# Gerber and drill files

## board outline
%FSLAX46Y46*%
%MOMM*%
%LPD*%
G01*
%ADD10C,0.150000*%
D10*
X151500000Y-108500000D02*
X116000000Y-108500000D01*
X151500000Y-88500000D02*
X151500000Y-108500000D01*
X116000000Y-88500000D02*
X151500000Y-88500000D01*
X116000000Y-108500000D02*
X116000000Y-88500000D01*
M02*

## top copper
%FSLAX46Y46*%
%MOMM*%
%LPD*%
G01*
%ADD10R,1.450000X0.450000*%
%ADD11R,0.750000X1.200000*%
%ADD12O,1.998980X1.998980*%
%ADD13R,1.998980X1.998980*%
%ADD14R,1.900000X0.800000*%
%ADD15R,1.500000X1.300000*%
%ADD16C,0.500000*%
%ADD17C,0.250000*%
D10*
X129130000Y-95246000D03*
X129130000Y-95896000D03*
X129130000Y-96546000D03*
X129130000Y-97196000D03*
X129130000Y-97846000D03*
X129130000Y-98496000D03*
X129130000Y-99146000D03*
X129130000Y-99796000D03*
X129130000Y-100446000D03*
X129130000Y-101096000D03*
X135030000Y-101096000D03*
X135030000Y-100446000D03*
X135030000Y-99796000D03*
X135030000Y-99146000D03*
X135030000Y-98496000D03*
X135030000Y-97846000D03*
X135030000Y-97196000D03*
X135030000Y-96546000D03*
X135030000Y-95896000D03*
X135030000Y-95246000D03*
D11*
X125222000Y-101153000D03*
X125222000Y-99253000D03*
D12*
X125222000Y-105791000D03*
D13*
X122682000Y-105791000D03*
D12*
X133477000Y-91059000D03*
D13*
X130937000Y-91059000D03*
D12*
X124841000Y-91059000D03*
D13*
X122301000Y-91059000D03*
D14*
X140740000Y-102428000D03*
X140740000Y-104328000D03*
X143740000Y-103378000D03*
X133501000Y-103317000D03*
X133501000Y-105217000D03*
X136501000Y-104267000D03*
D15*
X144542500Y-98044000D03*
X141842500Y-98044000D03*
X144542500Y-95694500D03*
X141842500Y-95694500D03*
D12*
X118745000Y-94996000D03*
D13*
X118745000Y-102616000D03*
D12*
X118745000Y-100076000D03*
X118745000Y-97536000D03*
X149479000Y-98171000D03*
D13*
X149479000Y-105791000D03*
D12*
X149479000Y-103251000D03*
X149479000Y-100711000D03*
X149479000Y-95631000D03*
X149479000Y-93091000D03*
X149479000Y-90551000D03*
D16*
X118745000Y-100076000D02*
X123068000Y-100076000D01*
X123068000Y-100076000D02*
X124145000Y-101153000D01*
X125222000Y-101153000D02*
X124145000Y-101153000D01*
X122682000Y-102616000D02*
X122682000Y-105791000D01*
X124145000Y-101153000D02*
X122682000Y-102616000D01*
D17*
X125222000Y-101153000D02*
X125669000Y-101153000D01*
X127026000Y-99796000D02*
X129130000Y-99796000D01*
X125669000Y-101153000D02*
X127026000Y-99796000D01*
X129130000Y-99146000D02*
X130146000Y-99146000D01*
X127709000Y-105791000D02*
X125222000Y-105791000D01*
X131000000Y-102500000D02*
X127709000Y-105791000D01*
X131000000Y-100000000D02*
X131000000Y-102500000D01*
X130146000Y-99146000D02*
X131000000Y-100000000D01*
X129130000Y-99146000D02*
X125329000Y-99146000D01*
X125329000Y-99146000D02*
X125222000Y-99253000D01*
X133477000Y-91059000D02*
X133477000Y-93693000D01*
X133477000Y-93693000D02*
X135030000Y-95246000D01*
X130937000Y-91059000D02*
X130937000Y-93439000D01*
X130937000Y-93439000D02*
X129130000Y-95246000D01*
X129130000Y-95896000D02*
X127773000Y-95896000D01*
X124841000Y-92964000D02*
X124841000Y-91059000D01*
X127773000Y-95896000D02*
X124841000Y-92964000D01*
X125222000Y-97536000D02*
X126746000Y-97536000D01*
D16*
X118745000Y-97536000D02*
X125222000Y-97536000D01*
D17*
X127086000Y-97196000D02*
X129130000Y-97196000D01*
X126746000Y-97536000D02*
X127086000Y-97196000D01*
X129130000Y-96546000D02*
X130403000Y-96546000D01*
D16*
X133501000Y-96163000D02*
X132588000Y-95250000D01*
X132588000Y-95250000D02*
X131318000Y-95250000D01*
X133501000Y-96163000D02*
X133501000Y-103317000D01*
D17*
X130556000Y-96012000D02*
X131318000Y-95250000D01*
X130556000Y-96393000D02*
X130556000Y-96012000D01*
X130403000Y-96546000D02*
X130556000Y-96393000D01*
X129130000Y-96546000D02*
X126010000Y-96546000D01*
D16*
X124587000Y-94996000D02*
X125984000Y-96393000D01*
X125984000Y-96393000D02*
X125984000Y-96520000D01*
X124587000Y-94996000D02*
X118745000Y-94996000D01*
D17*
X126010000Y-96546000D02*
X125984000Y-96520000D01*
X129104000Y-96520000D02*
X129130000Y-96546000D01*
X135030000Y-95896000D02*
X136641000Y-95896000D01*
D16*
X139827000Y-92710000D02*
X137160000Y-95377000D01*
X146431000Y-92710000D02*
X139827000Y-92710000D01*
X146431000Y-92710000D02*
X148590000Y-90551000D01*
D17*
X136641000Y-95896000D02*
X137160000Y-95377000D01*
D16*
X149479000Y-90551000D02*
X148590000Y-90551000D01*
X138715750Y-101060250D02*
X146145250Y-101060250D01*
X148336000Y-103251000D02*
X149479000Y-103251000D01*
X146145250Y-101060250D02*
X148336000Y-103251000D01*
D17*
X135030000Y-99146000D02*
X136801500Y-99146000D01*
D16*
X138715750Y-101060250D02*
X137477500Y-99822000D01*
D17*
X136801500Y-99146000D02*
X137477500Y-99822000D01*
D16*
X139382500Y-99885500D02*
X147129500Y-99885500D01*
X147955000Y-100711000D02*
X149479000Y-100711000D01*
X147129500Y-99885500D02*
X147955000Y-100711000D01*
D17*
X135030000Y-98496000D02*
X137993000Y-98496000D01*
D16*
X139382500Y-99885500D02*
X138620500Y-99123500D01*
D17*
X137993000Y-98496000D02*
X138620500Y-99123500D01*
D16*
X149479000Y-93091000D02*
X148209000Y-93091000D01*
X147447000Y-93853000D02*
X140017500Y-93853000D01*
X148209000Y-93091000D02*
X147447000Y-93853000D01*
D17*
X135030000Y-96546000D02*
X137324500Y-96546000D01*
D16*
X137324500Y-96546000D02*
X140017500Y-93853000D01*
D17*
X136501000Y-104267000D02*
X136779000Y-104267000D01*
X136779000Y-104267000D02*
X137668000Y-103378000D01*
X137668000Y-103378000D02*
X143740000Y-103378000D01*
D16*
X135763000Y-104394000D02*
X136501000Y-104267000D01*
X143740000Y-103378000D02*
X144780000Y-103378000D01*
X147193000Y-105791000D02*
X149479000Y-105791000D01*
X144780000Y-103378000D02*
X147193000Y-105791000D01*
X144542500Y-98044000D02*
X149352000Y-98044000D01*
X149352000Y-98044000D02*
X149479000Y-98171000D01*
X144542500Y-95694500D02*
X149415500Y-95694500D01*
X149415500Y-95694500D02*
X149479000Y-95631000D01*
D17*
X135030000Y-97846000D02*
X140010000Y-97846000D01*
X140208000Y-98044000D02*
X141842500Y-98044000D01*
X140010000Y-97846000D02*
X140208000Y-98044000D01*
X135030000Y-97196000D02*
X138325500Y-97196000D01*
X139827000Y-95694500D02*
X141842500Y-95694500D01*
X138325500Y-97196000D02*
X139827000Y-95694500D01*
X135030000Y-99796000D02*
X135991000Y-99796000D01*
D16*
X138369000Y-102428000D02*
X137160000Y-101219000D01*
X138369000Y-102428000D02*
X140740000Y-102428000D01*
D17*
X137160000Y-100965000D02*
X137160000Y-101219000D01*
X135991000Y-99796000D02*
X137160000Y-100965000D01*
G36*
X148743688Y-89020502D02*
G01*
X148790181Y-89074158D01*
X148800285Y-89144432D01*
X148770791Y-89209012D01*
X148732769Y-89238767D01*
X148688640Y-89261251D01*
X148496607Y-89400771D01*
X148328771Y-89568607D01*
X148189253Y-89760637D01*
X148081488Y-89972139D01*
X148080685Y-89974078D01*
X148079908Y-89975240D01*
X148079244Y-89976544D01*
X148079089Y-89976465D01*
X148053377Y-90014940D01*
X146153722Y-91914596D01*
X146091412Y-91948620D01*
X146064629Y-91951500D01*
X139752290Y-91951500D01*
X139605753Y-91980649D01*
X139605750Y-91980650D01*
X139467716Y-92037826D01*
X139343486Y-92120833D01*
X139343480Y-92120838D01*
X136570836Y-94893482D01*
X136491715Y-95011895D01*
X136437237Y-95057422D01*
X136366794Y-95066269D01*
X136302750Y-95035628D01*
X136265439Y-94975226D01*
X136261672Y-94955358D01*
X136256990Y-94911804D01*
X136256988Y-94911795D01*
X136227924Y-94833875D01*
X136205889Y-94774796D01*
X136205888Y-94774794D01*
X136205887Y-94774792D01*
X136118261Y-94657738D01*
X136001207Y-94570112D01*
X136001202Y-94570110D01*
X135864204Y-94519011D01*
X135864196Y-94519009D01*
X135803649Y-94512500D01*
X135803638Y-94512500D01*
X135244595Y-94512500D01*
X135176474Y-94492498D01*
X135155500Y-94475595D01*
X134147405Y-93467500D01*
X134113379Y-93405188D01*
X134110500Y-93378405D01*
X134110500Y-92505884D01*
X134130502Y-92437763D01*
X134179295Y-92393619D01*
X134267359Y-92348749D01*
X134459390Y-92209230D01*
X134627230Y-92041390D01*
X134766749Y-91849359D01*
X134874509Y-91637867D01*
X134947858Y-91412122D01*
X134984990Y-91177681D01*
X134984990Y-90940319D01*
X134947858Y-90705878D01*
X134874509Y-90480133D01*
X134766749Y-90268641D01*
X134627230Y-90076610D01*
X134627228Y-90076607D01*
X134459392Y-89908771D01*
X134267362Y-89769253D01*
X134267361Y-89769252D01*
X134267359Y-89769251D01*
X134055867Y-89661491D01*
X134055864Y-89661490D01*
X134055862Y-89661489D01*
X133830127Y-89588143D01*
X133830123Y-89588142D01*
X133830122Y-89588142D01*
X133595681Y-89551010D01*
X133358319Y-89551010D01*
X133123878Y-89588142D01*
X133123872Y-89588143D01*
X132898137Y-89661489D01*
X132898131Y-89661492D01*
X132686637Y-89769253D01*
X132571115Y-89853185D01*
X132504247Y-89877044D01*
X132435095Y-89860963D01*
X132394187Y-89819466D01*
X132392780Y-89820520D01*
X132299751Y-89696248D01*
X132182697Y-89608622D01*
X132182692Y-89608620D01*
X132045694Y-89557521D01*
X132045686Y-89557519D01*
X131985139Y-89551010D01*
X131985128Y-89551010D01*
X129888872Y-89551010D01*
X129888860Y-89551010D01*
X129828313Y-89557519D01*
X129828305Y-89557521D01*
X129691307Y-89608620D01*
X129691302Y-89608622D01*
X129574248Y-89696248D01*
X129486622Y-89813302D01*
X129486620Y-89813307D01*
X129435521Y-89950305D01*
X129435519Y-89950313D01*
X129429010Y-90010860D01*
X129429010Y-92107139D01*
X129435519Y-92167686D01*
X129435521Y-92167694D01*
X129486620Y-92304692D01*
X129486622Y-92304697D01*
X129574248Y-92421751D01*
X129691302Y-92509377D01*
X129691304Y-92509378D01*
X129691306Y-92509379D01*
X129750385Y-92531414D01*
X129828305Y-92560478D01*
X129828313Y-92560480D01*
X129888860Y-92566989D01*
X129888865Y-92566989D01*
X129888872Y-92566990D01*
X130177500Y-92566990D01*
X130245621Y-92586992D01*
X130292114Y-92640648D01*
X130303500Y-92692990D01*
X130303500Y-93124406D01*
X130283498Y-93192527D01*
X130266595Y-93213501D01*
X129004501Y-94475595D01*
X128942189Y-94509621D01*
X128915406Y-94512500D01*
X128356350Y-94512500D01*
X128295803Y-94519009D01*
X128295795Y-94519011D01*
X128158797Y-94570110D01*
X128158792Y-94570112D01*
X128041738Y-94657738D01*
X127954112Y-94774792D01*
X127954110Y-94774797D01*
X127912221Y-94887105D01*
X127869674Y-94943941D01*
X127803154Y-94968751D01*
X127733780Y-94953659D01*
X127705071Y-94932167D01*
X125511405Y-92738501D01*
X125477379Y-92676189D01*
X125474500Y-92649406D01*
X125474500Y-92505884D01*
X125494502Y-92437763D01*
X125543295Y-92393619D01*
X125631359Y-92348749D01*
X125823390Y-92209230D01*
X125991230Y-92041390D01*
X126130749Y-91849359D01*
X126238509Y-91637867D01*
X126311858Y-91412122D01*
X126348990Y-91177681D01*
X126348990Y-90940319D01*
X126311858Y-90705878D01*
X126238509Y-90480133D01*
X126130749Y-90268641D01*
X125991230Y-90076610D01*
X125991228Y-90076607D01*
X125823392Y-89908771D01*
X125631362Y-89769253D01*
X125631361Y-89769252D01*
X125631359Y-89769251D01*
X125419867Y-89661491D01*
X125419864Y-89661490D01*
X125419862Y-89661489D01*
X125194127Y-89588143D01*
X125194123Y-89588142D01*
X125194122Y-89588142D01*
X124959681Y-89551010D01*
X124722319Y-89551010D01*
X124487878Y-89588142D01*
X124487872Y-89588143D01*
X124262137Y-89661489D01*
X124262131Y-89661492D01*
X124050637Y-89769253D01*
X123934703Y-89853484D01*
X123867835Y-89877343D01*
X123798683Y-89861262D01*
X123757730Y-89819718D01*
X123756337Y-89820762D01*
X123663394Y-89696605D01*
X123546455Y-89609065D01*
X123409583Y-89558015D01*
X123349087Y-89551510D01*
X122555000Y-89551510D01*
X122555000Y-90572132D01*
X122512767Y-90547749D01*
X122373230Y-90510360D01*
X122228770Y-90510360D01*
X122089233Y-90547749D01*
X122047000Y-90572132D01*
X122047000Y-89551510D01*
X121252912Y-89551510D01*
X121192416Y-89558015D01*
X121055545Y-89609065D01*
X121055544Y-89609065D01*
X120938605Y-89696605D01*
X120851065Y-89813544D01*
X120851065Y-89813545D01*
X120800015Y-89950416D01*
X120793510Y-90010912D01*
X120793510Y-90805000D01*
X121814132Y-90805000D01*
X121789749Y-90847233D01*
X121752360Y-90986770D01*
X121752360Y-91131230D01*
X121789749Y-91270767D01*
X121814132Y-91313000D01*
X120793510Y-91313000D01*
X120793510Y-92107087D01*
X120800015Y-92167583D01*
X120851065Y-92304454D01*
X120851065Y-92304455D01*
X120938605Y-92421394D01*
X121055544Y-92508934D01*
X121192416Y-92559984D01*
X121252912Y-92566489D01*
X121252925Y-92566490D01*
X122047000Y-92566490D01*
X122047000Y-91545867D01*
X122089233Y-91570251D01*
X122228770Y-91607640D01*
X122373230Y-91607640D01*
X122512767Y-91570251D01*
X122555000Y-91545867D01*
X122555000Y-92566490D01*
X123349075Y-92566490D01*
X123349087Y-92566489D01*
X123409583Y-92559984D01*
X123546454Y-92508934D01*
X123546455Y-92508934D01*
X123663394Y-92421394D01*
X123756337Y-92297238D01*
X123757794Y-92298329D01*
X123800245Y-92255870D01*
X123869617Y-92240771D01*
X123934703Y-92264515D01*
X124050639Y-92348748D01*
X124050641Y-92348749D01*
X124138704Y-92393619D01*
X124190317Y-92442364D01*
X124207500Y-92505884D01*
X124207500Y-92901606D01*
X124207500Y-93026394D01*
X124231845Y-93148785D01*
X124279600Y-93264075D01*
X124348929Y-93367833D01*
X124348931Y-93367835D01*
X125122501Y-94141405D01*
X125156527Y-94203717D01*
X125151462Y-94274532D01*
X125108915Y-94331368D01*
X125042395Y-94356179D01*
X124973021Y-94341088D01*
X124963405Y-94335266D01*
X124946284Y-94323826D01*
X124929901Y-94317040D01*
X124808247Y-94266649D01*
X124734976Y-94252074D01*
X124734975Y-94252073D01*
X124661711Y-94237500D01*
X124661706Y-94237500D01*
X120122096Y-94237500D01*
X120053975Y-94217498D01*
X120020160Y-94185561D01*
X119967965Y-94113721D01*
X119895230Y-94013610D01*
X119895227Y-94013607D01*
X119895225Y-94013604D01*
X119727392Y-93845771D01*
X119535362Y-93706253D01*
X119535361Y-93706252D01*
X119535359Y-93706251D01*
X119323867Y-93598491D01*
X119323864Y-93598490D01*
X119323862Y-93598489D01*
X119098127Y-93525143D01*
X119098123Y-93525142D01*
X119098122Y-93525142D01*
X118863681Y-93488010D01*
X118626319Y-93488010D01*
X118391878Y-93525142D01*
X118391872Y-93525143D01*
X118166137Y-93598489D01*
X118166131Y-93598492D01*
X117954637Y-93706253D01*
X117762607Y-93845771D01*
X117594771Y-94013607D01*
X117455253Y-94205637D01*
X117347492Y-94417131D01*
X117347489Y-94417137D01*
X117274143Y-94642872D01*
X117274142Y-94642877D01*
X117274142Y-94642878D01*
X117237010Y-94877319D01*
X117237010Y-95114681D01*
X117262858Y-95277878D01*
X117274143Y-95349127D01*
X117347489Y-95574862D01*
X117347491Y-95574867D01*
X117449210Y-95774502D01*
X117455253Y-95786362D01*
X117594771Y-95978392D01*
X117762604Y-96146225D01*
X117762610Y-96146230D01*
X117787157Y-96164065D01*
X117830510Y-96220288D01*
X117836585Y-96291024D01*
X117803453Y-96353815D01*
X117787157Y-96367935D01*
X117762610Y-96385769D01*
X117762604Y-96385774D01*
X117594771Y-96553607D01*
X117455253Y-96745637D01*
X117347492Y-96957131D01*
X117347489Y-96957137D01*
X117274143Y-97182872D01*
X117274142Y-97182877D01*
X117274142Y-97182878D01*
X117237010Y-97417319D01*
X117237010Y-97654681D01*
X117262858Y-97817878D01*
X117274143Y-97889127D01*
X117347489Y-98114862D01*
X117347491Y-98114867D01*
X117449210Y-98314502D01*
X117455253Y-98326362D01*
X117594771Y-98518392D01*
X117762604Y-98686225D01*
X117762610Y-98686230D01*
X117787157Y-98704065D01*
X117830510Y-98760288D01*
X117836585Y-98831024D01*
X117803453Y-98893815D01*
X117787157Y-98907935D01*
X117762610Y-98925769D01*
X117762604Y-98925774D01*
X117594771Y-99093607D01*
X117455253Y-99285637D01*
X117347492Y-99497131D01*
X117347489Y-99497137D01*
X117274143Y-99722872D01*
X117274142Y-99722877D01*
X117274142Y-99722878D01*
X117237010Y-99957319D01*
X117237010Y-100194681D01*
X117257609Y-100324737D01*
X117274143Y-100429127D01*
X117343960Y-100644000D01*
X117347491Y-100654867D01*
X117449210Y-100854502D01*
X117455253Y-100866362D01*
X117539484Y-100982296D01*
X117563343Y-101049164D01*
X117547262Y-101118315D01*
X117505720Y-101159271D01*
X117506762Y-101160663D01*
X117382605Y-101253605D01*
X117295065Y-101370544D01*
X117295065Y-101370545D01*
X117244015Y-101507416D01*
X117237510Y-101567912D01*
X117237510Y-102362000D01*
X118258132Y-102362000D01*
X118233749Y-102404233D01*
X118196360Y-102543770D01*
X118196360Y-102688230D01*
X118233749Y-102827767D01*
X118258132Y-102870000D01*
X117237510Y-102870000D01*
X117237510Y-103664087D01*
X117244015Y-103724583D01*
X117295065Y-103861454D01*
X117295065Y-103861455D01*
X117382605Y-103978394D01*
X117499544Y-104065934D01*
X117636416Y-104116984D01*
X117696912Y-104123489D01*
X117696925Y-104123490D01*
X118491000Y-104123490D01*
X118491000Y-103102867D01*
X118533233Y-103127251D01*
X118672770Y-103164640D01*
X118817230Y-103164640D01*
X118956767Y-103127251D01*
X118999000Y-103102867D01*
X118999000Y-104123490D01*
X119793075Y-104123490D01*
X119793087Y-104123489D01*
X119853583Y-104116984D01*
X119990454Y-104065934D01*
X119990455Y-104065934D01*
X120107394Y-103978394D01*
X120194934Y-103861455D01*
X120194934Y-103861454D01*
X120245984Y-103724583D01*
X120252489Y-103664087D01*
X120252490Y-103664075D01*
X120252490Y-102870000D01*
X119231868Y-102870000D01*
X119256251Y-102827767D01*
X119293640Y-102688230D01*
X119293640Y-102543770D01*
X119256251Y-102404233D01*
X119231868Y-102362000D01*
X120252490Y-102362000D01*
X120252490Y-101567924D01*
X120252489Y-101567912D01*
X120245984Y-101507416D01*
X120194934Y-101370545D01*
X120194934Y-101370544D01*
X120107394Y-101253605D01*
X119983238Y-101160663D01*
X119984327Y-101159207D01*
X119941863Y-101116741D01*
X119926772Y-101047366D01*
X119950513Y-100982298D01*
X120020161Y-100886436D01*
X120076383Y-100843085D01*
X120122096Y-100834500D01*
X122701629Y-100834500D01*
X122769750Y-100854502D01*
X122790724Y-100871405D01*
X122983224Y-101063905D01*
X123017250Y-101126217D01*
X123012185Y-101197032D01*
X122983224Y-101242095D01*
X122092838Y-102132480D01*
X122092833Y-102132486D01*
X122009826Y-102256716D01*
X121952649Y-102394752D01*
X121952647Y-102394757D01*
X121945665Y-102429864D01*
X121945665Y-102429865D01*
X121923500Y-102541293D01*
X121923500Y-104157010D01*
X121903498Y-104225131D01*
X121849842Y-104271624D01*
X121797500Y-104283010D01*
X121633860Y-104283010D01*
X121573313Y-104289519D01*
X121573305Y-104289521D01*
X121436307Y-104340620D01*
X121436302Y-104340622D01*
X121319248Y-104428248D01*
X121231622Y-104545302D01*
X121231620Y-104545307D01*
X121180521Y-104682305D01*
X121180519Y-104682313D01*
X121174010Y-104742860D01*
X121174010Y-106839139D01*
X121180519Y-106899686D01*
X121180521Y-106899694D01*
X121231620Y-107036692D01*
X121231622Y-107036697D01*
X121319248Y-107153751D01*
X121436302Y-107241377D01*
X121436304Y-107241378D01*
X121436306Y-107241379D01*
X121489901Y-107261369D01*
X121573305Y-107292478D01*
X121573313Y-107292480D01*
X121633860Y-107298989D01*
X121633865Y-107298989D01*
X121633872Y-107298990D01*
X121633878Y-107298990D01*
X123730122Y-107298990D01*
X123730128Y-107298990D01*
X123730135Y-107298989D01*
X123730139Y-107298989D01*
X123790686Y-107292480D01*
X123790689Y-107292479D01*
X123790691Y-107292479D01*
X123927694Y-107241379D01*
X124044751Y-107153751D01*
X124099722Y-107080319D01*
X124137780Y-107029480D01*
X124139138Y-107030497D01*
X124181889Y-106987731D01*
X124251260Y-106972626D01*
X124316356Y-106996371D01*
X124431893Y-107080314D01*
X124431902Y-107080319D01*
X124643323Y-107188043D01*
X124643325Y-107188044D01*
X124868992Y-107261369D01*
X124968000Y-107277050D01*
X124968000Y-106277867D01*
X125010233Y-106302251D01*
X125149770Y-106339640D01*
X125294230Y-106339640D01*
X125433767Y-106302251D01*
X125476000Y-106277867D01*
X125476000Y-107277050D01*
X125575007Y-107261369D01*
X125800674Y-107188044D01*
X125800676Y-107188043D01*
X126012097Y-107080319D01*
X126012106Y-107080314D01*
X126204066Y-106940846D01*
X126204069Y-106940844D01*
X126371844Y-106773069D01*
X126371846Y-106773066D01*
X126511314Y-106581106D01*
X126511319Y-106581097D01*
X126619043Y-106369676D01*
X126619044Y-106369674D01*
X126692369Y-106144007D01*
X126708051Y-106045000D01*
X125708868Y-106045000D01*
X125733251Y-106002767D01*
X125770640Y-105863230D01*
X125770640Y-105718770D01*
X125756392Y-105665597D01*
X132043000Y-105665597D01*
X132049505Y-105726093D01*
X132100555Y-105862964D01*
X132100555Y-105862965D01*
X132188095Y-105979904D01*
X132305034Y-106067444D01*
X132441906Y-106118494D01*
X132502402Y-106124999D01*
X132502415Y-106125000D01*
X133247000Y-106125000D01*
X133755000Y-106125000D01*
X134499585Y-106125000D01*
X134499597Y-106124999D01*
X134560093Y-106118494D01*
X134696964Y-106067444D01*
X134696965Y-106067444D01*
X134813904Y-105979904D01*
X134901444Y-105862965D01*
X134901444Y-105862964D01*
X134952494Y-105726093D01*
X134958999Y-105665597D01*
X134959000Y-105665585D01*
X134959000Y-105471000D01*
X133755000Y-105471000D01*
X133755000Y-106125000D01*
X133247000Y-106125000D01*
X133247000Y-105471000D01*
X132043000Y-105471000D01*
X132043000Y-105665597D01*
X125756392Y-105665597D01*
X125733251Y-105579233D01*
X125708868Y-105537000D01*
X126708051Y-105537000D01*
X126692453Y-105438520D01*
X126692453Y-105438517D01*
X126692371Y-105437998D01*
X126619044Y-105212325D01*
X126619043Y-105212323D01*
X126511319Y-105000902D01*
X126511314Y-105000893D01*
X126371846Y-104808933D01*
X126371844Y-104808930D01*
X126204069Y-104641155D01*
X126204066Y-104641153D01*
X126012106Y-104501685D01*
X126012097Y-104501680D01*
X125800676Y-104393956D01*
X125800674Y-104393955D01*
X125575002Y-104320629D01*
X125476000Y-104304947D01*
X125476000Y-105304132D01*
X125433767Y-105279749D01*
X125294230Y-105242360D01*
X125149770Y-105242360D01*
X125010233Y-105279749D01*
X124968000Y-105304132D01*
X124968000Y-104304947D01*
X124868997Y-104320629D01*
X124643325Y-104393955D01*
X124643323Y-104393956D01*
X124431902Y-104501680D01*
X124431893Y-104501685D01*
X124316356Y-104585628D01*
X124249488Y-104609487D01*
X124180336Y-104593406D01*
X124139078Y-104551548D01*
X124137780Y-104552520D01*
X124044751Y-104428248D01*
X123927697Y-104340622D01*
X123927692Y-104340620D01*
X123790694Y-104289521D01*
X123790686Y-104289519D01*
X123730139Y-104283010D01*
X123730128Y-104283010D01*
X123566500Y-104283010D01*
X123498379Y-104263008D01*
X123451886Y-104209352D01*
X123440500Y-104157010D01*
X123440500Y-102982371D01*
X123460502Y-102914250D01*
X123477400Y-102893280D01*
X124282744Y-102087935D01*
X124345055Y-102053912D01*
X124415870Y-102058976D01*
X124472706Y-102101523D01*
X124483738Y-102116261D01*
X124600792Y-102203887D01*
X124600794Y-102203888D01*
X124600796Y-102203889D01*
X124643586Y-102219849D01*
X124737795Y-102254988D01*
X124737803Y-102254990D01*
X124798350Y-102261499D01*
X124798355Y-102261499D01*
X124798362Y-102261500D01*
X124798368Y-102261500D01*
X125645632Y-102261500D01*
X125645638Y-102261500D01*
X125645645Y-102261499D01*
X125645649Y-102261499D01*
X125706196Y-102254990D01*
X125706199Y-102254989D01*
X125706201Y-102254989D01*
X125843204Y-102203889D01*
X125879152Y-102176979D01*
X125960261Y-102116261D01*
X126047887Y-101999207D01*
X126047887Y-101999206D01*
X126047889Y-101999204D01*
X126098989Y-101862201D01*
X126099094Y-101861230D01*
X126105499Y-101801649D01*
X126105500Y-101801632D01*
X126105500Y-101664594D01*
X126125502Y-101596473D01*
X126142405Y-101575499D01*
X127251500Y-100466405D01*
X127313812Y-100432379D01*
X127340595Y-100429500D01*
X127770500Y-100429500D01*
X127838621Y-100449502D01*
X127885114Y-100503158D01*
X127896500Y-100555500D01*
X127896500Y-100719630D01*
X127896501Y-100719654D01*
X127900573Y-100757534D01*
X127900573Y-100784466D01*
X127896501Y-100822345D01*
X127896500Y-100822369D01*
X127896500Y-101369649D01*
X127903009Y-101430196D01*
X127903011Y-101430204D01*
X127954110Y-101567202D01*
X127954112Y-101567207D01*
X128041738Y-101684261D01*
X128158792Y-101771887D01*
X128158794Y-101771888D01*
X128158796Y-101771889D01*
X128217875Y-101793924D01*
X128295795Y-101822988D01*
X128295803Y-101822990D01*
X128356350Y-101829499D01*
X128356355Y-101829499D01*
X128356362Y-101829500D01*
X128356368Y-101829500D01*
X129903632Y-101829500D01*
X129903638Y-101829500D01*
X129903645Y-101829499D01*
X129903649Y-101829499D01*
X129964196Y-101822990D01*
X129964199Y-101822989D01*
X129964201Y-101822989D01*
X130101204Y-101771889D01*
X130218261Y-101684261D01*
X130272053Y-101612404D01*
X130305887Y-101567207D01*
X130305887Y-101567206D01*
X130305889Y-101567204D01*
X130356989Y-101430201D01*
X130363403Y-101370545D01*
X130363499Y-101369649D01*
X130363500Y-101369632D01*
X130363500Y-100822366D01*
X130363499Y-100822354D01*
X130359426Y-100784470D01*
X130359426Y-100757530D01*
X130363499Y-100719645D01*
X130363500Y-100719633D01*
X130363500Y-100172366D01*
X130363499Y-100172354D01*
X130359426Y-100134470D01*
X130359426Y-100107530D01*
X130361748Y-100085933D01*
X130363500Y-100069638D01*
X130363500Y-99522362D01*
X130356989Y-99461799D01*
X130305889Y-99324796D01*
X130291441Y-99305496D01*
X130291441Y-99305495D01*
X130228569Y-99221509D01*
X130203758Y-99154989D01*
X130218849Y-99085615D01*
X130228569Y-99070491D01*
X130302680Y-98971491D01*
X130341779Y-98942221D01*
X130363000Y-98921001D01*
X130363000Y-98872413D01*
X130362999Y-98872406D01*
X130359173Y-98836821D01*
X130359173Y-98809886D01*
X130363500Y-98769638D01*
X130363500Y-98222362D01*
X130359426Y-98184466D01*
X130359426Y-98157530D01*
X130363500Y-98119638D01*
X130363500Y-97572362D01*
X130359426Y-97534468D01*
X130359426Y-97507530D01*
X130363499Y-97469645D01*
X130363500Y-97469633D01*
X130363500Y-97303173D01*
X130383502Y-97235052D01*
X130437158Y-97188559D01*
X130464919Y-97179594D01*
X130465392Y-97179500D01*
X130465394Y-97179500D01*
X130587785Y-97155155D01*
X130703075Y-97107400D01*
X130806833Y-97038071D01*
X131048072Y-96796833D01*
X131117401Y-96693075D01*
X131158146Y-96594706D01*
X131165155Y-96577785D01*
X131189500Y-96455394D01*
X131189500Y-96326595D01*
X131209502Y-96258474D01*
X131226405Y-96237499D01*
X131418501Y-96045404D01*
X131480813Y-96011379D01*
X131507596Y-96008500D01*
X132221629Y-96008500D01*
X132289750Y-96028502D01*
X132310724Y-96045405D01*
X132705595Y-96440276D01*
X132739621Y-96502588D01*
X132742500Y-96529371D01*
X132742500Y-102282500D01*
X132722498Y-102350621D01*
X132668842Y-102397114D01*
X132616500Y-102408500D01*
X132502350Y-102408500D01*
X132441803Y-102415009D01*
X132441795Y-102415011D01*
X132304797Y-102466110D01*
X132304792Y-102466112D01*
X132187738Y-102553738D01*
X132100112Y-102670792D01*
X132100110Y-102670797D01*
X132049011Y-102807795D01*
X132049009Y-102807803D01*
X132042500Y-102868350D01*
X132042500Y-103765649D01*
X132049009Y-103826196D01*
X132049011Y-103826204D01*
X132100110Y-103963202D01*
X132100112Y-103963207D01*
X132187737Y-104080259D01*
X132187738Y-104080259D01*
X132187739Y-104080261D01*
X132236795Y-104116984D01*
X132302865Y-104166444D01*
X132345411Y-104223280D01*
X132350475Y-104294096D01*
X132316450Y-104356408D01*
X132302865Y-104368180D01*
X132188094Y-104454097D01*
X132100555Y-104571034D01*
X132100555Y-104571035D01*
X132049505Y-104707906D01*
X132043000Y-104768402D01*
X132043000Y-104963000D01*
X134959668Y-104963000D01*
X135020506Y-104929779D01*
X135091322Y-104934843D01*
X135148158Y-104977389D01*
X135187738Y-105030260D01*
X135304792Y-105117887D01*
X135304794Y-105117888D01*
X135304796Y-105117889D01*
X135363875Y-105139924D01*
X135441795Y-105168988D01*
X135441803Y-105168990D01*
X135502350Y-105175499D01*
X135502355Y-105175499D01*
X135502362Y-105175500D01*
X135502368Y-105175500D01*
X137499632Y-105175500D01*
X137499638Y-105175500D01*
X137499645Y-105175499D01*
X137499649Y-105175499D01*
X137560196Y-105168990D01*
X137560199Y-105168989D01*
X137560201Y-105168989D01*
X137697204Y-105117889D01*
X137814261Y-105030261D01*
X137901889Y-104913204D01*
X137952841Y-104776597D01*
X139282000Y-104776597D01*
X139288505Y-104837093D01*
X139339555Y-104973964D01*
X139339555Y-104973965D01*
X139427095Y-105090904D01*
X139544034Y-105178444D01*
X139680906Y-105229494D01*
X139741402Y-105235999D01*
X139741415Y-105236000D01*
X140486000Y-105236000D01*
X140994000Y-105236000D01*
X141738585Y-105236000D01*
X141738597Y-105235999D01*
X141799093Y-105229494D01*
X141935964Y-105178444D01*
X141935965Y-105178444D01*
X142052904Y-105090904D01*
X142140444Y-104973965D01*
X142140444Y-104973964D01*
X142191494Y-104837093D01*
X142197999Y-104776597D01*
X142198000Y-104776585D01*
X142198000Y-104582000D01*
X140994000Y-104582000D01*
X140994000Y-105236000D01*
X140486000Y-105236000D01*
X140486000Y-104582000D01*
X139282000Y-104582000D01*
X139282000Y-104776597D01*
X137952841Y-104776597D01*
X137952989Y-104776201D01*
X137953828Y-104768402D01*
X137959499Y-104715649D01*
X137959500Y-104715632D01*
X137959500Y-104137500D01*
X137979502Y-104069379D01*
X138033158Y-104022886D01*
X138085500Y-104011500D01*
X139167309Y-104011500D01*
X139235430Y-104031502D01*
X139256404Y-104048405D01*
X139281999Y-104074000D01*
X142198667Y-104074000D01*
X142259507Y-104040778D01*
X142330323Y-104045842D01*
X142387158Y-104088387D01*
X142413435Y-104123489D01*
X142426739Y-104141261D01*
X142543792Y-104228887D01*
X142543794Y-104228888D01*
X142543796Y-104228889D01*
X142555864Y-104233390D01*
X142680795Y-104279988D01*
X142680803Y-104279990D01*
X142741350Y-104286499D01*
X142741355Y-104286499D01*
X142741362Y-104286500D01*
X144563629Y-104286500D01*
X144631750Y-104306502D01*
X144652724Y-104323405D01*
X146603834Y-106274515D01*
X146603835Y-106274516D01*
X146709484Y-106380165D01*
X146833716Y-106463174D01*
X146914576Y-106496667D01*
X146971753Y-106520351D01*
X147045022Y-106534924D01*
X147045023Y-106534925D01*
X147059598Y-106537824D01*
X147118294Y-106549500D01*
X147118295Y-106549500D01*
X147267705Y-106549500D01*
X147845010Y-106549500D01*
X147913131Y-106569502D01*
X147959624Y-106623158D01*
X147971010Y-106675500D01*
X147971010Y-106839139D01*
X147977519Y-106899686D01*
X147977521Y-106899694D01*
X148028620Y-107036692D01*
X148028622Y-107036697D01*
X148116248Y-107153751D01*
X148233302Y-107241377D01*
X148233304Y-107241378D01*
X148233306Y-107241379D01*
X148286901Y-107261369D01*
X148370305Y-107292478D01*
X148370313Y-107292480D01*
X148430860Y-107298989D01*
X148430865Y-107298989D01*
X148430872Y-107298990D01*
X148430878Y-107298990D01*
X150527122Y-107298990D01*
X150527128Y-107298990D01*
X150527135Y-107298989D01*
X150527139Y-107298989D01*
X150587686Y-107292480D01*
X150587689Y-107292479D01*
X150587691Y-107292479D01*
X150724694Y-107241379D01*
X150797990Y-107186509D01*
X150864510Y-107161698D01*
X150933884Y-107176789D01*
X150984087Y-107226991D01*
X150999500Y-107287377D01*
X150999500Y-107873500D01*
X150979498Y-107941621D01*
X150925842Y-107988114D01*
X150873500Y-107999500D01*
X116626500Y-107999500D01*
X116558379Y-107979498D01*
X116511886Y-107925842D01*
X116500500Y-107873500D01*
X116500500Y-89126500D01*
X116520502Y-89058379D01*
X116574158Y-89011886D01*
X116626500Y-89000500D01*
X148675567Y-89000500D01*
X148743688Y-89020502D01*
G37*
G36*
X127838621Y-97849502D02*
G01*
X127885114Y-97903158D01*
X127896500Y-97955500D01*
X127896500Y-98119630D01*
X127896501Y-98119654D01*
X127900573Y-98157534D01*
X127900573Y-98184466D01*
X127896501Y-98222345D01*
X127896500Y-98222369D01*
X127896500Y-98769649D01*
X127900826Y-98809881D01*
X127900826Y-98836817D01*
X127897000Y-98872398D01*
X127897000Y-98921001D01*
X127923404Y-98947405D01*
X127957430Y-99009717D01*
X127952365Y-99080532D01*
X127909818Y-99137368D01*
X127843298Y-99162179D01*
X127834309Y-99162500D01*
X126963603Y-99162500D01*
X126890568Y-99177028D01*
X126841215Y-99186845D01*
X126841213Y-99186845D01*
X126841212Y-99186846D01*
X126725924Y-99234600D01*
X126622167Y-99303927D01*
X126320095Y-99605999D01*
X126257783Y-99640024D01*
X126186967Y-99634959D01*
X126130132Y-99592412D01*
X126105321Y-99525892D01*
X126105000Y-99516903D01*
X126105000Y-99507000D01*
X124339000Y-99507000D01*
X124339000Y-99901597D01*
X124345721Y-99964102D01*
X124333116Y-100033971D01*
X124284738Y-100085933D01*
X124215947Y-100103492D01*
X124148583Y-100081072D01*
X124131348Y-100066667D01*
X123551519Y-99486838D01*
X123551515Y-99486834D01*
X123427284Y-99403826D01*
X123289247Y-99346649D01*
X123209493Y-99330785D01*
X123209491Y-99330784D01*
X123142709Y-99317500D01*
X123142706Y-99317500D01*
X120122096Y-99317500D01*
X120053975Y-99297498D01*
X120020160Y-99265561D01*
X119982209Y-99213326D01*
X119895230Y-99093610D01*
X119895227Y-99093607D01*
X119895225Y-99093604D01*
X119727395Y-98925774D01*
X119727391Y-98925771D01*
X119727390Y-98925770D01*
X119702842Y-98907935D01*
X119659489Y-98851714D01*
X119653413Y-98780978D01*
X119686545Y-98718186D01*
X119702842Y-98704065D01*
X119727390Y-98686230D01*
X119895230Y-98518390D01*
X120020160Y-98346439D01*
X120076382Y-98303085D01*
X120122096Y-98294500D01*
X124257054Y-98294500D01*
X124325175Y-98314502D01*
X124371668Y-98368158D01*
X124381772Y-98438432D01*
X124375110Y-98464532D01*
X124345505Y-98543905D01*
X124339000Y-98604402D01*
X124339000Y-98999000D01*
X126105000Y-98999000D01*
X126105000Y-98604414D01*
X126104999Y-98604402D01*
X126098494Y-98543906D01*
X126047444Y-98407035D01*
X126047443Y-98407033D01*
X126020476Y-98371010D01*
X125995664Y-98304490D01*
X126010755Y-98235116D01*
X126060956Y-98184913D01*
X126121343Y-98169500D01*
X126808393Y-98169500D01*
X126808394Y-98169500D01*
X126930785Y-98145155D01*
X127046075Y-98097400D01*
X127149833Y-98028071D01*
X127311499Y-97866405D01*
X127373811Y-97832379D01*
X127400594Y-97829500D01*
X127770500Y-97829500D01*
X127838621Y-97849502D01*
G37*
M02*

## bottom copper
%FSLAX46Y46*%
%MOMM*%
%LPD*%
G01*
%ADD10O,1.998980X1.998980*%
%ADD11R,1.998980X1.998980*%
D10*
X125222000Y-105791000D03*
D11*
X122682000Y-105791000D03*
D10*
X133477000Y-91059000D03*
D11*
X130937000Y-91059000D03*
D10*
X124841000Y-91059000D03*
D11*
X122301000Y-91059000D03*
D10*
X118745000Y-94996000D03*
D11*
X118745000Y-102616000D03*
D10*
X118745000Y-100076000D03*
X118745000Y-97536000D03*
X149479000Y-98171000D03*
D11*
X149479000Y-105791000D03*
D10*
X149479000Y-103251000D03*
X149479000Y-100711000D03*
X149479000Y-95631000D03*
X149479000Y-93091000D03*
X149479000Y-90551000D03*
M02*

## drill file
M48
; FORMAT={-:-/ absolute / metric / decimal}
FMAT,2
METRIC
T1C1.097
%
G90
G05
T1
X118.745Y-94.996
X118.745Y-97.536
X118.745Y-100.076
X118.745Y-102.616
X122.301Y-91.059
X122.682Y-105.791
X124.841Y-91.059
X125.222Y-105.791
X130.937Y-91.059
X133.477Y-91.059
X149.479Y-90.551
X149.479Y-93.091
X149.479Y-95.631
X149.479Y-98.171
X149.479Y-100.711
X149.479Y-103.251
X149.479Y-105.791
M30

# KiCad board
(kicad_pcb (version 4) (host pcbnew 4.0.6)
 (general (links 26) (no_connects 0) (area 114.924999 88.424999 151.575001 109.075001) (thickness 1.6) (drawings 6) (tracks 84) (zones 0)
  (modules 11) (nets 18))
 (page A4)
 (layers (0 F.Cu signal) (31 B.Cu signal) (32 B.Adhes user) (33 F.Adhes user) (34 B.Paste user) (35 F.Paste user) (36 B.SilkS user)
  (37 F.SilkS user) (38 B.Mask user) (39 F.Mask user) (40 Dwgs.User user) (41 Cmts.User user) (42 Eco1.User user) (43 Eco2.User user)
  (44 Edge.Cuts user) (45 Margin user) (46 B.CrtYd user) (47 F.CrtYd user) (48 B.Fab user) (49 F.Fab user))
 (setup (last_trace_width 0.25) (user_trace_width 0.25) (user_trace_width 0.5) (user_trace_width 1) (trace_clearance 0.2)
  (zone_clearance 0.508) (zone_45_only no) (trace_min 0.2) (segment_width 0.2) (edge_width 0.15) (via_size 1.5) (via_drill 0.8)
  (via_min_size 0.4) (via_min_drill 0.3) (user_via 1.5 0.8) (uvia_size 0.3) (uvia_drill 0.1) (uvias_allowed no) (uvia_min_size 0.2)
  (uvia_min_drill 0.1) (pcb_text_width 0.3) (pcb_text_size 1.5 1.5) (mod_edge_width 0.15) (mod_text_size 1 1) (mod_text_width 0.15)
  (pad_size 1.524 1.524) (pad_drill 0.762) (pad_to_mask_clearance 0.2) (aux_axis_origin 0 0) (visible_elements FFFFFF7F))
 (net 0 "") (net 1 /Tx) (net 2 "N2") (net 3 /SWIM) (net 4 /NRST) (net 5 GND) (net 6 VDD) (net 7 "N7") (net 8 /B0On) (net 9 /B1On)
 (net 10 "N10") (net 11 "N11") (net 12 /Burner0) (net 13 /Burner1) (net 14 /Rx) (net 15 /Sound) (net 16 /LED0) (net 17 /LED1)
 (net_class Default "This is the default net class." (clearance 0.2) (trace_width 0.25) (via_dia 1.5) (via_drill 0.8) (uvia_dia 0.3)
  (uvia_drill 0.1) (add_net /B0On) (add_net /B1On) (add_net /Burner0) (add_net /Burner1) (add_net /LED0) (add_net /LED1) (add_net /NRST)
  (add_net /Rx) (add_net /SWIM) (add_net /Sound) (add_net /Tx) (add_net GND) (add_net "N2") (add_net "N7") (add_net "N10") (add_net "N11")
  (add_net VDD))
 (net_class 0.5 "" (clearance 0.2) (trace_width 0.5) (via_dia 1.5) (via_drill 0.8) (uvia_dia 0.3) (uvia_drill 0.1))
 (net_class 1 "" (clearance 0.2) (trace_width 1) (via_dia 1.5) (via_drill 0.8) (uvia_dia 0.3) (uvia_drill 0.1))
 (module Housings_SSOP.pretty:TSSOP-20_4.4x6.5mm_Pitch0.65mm (layer F.Cu) (at 132.08 98.171)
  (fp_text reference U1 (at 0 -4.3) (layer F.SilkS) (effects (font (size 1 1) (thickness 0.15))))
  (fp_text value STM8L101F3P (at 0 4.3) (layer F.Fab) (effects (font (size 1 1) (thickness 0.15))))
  (pad 1 smd rect (at -2.95 -2.925) (size 1.45 0.45) (layers F.Cu F.Paste F.Mask) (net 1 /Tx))
  (pad 2 smd rect (at -2.95 -2.275) (size 1.45 0.45) (layers F.Cu F.Paste F.Mask) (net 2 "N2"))
  (pad 3 smd rect (at -2.95 -1.625) (size 1.45 0.45) (layers F.Cu F.Paste F.Mask) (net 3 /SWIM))
  (pad 4 smd rect (at -2.95 -0.975) (size 1.45 0.45) (layers F.Cu F.Paste F.Mask) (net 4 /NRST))
  (pad 5 smd rect (at -2.95 -0.325) (size 1.45 0.45) (layers F.Cu F.Paste F.Mask))
  (pad 6 smd rect (at -2.95 0.325) (size 1.45 0.45) (layers F.Cu F.Paste F.Mask))
  (pad 7 smd rect (at -2.95 0.975) (size 1.45 0.45) (layers F.Cu F.Paste F.Mask) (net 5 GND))
  (pad 8 smd rect (at -2.95 1.625) (size 1.45 0.45) (layers F.Cu F.Paste F.Mask) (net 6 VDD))
  (pad 9 smd rect (at -2.95 2.275) (size 1.45 0.45) (layers F.Cu F.Paste F.Mask))
  (pad 10 smd rect (at -2.95 2.925) (size 1.45 0.45) (layers F.Cu F.Paste F.Mask))
  (pad 11 smd rect (at 2.95 2.925) (size 1.45 0.45) (layers F.Cu F.Paste F.Mask))
  (pad 12 smd rect (at 2.95 2.275) (size 1.45 0.45) (layers F.Cu F.Paste F.Mask))
  (pad 13 smd rect (at 2.95 1.625) (size 1.45 0.45) (layers F.Cu F.Paste F.Mask) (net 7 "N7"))
  (pad 14 smd rect (at 2.95 0.975) (size 1.45 0.45) (layers F.Cu F.Paste F.Mask) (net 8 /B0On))
  (pad 15 smd rect (at 2.95 0.325) (size 1.45 0.45) (layers F.Cu F.Paste F.Mask) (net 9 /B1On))
  (pad 16 smd rect (at 2.95 -0.325) (size 1.45 0.45) (layers F.Cu F.Paste F.Mask) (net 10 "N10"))
  (pad 17 smd rect (at 2.95 -0.975) (size 1.45 0.45) (layers F.Cu F.Paste F.Mask) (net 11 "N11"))
  (pad 18 smd rect (at 2.95 -1.625) (size 1.45 0.45) (layers F.Cu F.Paste F.Mask) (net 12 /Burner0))
  (pad 19 smd rect (at 2.95 -2.275) (size 1.45 0.45) (layers F.Cu F.Paste F.Mask) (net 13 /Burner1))
  (pad 20 smd rect (at 2.95 -2.925) (size 1.45 0.45) (layers F.Cu F.Paste F.Mask) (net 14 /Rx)))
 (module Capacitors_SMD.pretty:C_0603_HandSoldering (layer F.Cu) (at 125.222 100.203 90)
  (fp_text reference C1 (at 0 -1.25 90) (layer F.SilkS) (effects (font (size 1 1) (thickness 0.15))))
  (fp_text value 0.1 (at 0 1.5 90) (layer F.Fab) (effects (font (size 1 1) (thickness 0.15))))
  (pad 1 smd rect (at -0.95 0 90) (size 1.2 0.75) (layers F.Cu F.Paste F.Mask) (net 6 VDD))
  (pad 2 smd rect (at 0.95 0 90) (size 1.2 0.75) (layers F.Cu F.Paste F.Mask) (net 5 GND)))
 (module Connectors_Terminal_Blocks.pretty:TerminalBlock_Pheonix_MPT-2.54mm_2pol (layer B.Cu) (at 122.682 105.791)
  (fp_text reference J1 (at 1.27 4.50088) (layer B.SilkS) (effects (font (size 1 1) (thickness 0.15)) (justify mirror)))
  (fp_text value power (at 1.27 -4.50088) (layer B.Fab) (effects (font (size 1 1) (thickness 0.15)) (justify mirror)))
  (pad 2 thru_hole oval (at 2.54 0) (size 1.99898 1.99898) (drill 1.09728) (layers *.Cu *.Mask) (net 5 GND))
  (pad 1 thru_hole rect (at 0 0) (size 1.99898 1.99898) (drill 1.09728) (layers *.Cu *.Mask) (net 6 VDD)))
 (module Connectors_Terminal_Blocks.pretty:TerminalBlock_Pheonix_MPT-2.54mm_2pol (layer B.Cu) (at 130.937 91.059)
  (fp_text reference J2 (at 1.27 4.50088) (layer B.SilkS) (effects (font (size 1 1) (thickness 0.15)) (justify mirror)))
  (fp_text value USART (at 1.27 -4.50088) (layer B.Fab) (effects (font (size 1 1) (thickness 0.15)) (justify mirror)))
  (pad 2 thru_hole oval (at 2.54 0) (size 1.99898 1.99898) (drill 1.09728) (layers *.Cu *.Mask) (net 14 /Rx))
  (pad 1 thru_hole rect (at 0 0) (size 1.99898 1.99898) (drill 1.09728) (layers *.Cu *.Mask) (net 1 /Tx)))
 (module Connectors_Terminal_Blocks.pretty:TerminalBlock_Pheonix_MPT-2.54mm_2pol (layer B.Cu) (at 122.301 91.059)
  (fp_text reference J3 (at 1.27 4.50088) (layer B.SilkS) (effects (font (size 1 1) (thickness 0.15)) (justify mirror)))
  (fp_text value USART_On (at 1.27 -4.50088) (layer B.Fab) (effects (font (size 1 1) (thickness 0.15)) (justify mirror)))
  (pad 2 thru_hole oval (at 2.54 0) (size 1.99898 1.99898) (drill 1.09728) (layers *.Cu *.Mask) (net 2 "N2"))
  (pad 1 thru_hole rect (at 0 0) (size 1.99898 1.99898) (drill 1.09728) (layers *.Cu *.Mask) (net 5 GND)))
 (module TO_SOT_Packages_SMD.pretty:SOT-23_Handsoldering (layer F.Cu) (at 142.24 103.378)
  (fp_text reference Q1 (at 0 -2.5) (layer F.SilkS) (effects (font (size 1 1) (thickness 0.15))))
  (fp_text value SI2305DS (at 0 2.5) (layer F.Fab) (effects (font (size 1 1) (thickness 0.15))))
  (pad 1 smd rect (at -1.5 -0.95) (size 1.9 0.8) (layers F.Cu F.Paste F.Mask) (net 7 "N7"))
  (pad 2 smd rect (at -1.5 0.95) (size 1.9 0.8) (layers F.Cu F.Paste F.Mask) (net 5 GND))
  (pad 3 smd rect (at 1.5 0) (size 1.9 0.8) (layers F.Cu F.Paste F.Mask) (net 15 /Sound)))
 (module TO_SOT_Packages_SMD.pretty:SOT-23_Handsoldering (layer F.Cu) (at 135.001 104.267)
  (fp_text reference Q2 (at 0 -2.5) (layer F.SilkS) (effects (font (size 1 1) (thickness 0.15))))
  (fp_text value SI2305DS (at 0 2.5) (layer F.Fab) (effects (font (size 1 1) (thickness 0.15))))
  (pad 1 smd rect (at -1.5 -0.95) (size 1.9 0.8) (layers F.Cu F.Paste F.Mask) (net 3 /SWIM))
  (pad 2 smd rect (at -1.5 0.95) (size 1.9 0.8) (layers F.Cu F.Paste F.Mask) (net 5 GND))
  (pad 3 smd rect (at 1.5 0) (size 1.9 0.8) (layers F.Cu F.Paste F.Mask) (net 15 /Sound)))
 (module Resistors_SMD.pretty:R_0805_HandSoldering (layer F.Cu) (at 143.1925 98.044 180)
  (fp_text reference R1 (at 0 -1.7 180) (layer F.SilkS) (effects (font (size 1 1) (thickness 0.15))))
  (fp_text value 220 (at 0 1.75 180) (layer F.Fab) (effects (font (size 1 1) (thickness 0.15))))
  (pad 1 smd rect (at -1.35 0 180) (size 1.5 1.3) (layers F.Cu F.Paste F.Mask) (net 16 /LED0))
  (pad 2 smd rect (at 1.35 0 180) (size 1.5 1.3) (layers F.Cu F.Paste F.Mask) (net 10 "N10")))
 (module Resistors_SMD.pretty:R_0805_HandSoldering (layer F.Cu) (at 143.1925 95.6945 180)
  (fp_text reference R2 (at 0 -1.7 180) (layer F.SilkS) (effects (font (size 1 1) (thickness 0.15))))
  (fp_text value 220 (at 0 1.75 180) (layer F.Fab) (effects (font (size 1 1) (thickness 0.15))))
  (pad 1 smd rect (at -1.35 0 180) (size 1.5 1.3) (layers F.Cu F.Paste F.Mask) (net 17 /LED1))
  (pad 2 smd rect (at 1.35 0 180) (size 1.5 1.3) (layers F.Cu F.Paste F.Mask) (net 11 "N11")))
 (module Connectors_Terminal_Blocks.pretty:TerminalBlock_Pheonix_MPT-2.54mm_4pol (layer B.Cu) (at 118.745 102.616 90)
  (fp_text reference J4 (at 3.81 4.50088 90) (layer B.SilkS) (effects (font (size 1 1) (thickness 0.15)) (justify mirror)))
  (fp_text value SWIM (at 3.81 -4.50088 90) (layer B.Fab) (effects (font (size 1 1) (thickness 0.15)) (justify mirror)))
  (pad 4 thru_hole oval (at 7.62 0 270) (size 1.99898 1.99898) (drill 1.09728) (layers *.Cu *.Mask) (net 3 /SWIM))
  (pad 1 thru_hole rect (at 0 0 270) (size 1.99898 1.99898) (drill 1.09728) (layers *.Cu *.Mask) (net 5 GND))
  (pad 2 thru_hole oval (at 2.54 0 270) (size 1.99898 1.99898) (drill 1.09728) (layers *.Cu *.Mask) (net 6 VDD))
  (pad 3 thru_hole oval (at 5.08 0 270) (size 1.99898 1.99898) (drill 1.09728) (layers *.Cu *.Mask) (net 4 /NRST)))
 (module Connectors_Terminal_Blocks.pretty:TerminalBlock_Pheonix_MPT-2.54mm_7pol (layer B.Cu) (at 149.479 105.791 90)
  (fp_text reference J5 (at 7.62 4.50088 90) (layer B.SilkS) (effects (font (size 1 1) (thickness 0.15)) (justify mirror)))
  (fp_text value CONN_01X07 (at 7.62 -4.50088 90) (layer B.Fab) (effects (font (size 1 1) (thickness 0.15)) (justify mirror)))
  (pad 4 thru_hole oval (at 7.62 0 270) (size 1.99898 1.99898) (drill 1.09728) (layers *.Cu *.Mask) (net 16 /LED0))
  (pad 1 thru_hole rect (at 0 0 270) (size 1.99898 1.99898) (drill 1.09728) (layers *.Cu *.Mask) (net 15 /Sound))
  (pad 2 thru_hole oval (at 2.54 0 270) (size 1.99898 1.99898) (drill 1.09728) (layers *.Cu *.Mask) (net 8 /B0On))
  (pad 3 thru_hole oval (at 5.08 0 270) (size 1.99898 1.99898) (drill 1.09728) (layers *.Cu *.Mask) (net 9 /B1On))
  (pad 5 thru_hole oval (at 10.16 0 270) (size 1.99898 1.99898) (drill 1.09728) (layers *.Cu *.Mask) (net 17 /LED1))
  (pad 6 thru_hole oval (at 12.7 0 270) (size 1.99898 1.99898) (drill 1.09728) (layers *.Cu *.Mask) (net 12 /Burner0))
  (pad 7 thru_hole oval (at 15.24 0 270) (size 1.99898 1.99898) (drill 1.09728) (layers *.Cu *.Mask) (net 13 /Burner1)))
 (gr_line (start 151.5 108.5) (end 116 108.5) (angle 90) (layer Edge.Cuts) (width 0.15))
 (gr_line (start 151.5 88.5) (end 151.5 108.5) (angle 90) (layer Edge.Cuts) (width 0.15))
 (gr_line (start 116 88.5) (end 151.5 88.5) (angle 90) (layer Edge.Cuts) (width 0.15))
 (gr_line (start 116 108.5) (end 116 88.5) (angle 90) (layer Edge.Cuts) (width 0.15))
 (segment (start 118.745 100.076) (end 123.068 100.076) (width 0.5) (layer F.Cu) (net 6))
 (segment (start 123.068 100.076) (end 124.145 101.153) (width 0.5) (layer F.Cu) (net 6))
 (segment (start 125.222 101.153) (end 124.145 101.153) (width 0.5) (layer F.Cu) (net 6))
 (segment (start 122.682 102.616) (end 122.682 105.791) (width 0.5) (layer F.Cu) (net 6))
 (segment (start 124.145 101.153) (end 122.682 102.616) (width 0.5) (layer F.Cu) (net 6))
 (segment (start 125.222 101.153) (end 125.669 101.153) (width 0.25) (layer F.Cu) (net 6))
 (segment (start 127.026 99.796) (end 129.13 99.796) (width 0.25) (layer F.Cu) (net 6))
 (segment (start 125.669 101.153) (end 127.026 99.796) (width 0.25) (layer F.Cu) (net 6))
 (segment (start 129.13 99.146) (end 130.146 99.146) (width 0.25) (layer F.Cu) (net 5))
 (segment (start 127.709 105.791) (end 125.222 105.791) (width 0.25) (layer F.Cu) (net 5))
 (segment (start 131 102.5) (end 127.709 105.791) (width 0.25) (layer F.Cu) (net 5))
 (segment (start 131 100) (end 131 102.5) (width 0.25) (layer F.Cu) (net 5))
 (segment (start 130.146 99.146) (end 131 100) (width 0.25) (layer F.Cu) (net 5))
 (segment (start 129.13 99.146) (end 125.329 99.146) (width 0.25) (layer F.Cu) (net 5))
 (segment (start 125.329 99.146) (end 125.222 99.253) (width 0.25) (layer F.Cu) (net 5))
 (segment (start 133.477 91.059) (end 133.477 93.693) (width 0.25) (layer F.Cu) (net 14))
 (segment (start 133.477 93.693) (end 135.03 95.246) (width 0.25) (layer F.Cu) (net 14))
 (segment (start 130.937 91.059) (end 130.937 93.439) (width 0.25) (layer F.Cu) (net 1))
 (segment (start 130.937 93.439) (end 129.13 95.246) (width 0.25) (layer F.Cu) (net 1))
 (segment (start 129.13 95.896) (end 127.773 95.896) (width 0.25) (layer F.Cu) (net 2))
 (segment (start 124.841 92.964) (end 124.841 91.059) (width 0.25) (layer F.Cu) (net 2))
 (segment (start 127.773 95.896) (end 124.841 92.964) (width 0.25) (layer F.Cu) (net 2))
 (segment (start 125.222 97.536) (end 126.746 97.536) (width 0.25) (layer F.Cu) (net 4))
 (segment (start 118.745 97.536) (end 125.222 97.536) (width 0.5) (layer F.Cu) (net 4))
 (segment (start 127.086 97.196) (end 129.13 97.196) (width 0.25) (layer F.Cu) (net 4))
 (segment (start 126.746 97.536) (end 127.086 97.196) (width 0.25) (layer F.Cu) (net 4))
 (segment (start 129.13 96.546) (end 130.403 96.546) (width 0.25) (layer F.Cu) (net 3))
 (segment (start 133.501 96.163) (end 132.588 95.25) (width 0.5) (layer F.Cu) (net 3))
 (segment (start 132.588 95.25) (end 131.318 95.25) (width 0.5) (layer F.Cu) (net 3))
 (segment (start 133.501 96.163) (end 133.501 103.317) (width 0.5) (layer F.Cu) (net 3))
 (segment (start 130.556 96.012) (end 131.318 95.25) (width 0.25) (layer F.Cu) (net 3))
 (segment (start 130.556 96.393) (end 130.556 96.012) (width 0.25) (layer F.Cu) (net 3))
 (segment (start 130.403 96.546) (end 130.556 96.393) (width 0.25) (layer F.Cu) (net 3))
 (segment (start 129.13 96.546) (end 126.01 96.546) (width 0.25) (layer F.Cu) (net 3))
 (segment (start 124.587 94.996) (end 125.984 96.393) (width 0.5) (layer F.Cu) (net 3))
 (segment (start 125.984 96.393) (end 125.984 96.52) (width 0.5) (layer F.Cu) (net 3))
 (segment (start 124.587 94.996) (end 118.745 94.996) (width 0.5) (layer F.Cu) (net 3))
 (segment (start 126.01 96.546) (end 125.984 96.52) (width 0.25) (layer F.Cu) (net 3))
 (segment (start 129.104 96.52) (end 129.13 96.546) (width 0.25) (layer F.Cu) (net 3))
 (segment (start 135.03 95.896) (end 136.641 95.896) (width 0.25) (layer F.Cu) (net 13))
 (segment (start 139.827 92.71) (end 137.16 95.377) (width 0.5) (layer F.Cu) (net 13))
 (segment (start 146.431 92.71) (end 139.827 92.71) (width 0.5) (layer F.Cu) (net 13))
 (segment (start 146.431 92.71) (end 148.59 90.551) (width 0.5) (layer F.Cu) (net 13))
 (segment (start 136.641 95.896) (end 137.16 95.377) (width 0.25) (layer F.Cu) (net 13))
 (segment (start 149.479 90.551) (end 148.59 90.551) (width 0.5) (layer F.Cu) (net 13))
 (segment (start 138.71575 101.06025) (end 146.14525 101.06025) (width 0.5) (layer F.Cu) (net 8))
 (segment (start 148.336 103.251) (end 149.479 103.251) (width 0.5) (layer F.Cu) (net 8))
 (segment (start 146.14525 101.06025) (end 148.336 103.251) (width 0.5) (layer F.Cu) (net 8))
 (segment (start 135.03 99.146) (end 136.8015 99.146) (width 0.25) (layer F.Cu) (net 8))
 (segment (start 138.71575 101.06025) (end 137.4775 99.822) (width 0.5) (layer F.Cu) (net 8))
 (segment (start 136.8015 99.146) (end 137.4775 99.822) (width 0.25) (layer F.Cu) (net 8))
 (segment (start 139.3825 99.8855) (end 147.1295 99.8855) (width 0.5) (layer F.Cu) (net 9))
 (segment (start 147.955 100.711) (end 149.479 100.711) (width 0.5) (layer F.Cu) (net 9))
 (segment (start 147.1295 99.8855) (end 147.955 100.711) (width 0.5) (layer F.Cu) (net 9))
 (segment (start 135.03 98.496) (end 137.993 98.496) (width 0.25) (layer F.Cu) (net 9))
 (segment (start 139.3825 99.8855) (end 138.6205 99.1235) (width 0.5) (layer F.Cu) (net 9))
 (segment (start 137.993 98.496) (end 138.6205 99.1235) (width 0.25) (layer F.Cu) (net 9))
 (segment (start 149.479 93.091) (end 148.209 93.091) (width 0.5) (layer F.Cu) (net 12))
 (segment (start 147.447 93.853) (end 140.0175 93.853) (width 0.5) (layer F.Cu) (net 12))
 (segment (start 148.209 93.091) (end 147.447 93.853) (width 0.5) (layer F.Cu) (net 12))
 (segment (start 135.03 96.546) (end 137.3245 96.546) (width 0.25) (layer F.Cu) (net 12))
 (segment (start 137.3245 96.546) (end 140.0175 93.853) (width 0.5) (layer F.Cu) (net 12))
 (segment (start 136.501 104.267) (end 136.779 104.267) (width 0.25) (layer F.Cu) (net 15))
 (segment (start 136.779 104.267) (end 137.668 103.378) (width 0.25) (layer F.Cu) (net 15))
 (segment (start 137.668 103.378) (end 143.74 103.378) (width 0.25) (layer F.Cu) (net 15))
 (segment (start 135.763 104.394) (end 136.501 104.267) (width 0.5) (layer F.Cu) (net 15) (status 20))
 (segment (start 143.74 103.378) (end 144.78 103.378) (width 0.5) (layer F.Cu) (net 15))
 (segment (start 147.193 105.791) (end 149.479 105.791) (width 0.5) (layer F.Cu) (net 15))
 (segment (start 144.78 103.378) (end 147.193 105.791) (width 0.5) (layer F.Cu) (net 15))
 (segment (start 144.5425 98.044) (end 149.352 98.044) (width 0.5) (layer F.Cu) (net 16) (status 20))
 (segment (start 149.352 98.044) (end 149.479 98.171) (width 0.5) (layer F.Cu) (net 16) (status 30))
 (segment (start 144.5425 95.6945) (end 149.4155 95.6945) (width 0.5) (layer F.Cu) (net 17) (status 20))
 (segment (start 149.4155 95.6945) (end 149.479 95.631) (width 0.5) (layer F.Cu) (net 17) (status 30))
 (segment (start 135.03 97.846) (end 140.01 97.846) (width 0.25) (layer F.Cu) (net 10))
 (segment (start 140.208 98.044) (end 141.8425 98.044) (width 0.25) (layer F.Cu) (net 10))
 (segment (start 140.01 97.846) (end 140.208 98.044) (width 0.25) (layer F.Cu) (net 10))
 (segment (start 135.03 97.196) (end 138.3255 97.196) (width 0.25) (layer F.Cu) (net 11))
 (segment (start 139.827 95.6945) (end 141.8425 95.6945) (width 0.25) (layer F.Cu) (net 11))
 (segment (start 138.3255 97.196) (end 139.827 95.6945) (width 0.25) (layer F.Cu) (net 11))
 (segment (start 135.03 99.796) (end 135.991 99.796) (width 0.25) (layer F.Cu) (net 7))
 (segment (start 138.369 102.428) (end 137.16 101.219) (width 0.5) (layer F.Cu) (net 7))
 (segment (start 138.369 102.428) (end 140.74 102.428) (width 0.5) (layer F.Cu) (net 7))
 (segment (start 137.16 100.965) (end 137.16 101.219) (width 0.25) (layer F.Cu) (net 7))
 (segment (start 135.991 99.796) (end 137.16 100.965) (width 0.25) (layer F.Cu) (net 7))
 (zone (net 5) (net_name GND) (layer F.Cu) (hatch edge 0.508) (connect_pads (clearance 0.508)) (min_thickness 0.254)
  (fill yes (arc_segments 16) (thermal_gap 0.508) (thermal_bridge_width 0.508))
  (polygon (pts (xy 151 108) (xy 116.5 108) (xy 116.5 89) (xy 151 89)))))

